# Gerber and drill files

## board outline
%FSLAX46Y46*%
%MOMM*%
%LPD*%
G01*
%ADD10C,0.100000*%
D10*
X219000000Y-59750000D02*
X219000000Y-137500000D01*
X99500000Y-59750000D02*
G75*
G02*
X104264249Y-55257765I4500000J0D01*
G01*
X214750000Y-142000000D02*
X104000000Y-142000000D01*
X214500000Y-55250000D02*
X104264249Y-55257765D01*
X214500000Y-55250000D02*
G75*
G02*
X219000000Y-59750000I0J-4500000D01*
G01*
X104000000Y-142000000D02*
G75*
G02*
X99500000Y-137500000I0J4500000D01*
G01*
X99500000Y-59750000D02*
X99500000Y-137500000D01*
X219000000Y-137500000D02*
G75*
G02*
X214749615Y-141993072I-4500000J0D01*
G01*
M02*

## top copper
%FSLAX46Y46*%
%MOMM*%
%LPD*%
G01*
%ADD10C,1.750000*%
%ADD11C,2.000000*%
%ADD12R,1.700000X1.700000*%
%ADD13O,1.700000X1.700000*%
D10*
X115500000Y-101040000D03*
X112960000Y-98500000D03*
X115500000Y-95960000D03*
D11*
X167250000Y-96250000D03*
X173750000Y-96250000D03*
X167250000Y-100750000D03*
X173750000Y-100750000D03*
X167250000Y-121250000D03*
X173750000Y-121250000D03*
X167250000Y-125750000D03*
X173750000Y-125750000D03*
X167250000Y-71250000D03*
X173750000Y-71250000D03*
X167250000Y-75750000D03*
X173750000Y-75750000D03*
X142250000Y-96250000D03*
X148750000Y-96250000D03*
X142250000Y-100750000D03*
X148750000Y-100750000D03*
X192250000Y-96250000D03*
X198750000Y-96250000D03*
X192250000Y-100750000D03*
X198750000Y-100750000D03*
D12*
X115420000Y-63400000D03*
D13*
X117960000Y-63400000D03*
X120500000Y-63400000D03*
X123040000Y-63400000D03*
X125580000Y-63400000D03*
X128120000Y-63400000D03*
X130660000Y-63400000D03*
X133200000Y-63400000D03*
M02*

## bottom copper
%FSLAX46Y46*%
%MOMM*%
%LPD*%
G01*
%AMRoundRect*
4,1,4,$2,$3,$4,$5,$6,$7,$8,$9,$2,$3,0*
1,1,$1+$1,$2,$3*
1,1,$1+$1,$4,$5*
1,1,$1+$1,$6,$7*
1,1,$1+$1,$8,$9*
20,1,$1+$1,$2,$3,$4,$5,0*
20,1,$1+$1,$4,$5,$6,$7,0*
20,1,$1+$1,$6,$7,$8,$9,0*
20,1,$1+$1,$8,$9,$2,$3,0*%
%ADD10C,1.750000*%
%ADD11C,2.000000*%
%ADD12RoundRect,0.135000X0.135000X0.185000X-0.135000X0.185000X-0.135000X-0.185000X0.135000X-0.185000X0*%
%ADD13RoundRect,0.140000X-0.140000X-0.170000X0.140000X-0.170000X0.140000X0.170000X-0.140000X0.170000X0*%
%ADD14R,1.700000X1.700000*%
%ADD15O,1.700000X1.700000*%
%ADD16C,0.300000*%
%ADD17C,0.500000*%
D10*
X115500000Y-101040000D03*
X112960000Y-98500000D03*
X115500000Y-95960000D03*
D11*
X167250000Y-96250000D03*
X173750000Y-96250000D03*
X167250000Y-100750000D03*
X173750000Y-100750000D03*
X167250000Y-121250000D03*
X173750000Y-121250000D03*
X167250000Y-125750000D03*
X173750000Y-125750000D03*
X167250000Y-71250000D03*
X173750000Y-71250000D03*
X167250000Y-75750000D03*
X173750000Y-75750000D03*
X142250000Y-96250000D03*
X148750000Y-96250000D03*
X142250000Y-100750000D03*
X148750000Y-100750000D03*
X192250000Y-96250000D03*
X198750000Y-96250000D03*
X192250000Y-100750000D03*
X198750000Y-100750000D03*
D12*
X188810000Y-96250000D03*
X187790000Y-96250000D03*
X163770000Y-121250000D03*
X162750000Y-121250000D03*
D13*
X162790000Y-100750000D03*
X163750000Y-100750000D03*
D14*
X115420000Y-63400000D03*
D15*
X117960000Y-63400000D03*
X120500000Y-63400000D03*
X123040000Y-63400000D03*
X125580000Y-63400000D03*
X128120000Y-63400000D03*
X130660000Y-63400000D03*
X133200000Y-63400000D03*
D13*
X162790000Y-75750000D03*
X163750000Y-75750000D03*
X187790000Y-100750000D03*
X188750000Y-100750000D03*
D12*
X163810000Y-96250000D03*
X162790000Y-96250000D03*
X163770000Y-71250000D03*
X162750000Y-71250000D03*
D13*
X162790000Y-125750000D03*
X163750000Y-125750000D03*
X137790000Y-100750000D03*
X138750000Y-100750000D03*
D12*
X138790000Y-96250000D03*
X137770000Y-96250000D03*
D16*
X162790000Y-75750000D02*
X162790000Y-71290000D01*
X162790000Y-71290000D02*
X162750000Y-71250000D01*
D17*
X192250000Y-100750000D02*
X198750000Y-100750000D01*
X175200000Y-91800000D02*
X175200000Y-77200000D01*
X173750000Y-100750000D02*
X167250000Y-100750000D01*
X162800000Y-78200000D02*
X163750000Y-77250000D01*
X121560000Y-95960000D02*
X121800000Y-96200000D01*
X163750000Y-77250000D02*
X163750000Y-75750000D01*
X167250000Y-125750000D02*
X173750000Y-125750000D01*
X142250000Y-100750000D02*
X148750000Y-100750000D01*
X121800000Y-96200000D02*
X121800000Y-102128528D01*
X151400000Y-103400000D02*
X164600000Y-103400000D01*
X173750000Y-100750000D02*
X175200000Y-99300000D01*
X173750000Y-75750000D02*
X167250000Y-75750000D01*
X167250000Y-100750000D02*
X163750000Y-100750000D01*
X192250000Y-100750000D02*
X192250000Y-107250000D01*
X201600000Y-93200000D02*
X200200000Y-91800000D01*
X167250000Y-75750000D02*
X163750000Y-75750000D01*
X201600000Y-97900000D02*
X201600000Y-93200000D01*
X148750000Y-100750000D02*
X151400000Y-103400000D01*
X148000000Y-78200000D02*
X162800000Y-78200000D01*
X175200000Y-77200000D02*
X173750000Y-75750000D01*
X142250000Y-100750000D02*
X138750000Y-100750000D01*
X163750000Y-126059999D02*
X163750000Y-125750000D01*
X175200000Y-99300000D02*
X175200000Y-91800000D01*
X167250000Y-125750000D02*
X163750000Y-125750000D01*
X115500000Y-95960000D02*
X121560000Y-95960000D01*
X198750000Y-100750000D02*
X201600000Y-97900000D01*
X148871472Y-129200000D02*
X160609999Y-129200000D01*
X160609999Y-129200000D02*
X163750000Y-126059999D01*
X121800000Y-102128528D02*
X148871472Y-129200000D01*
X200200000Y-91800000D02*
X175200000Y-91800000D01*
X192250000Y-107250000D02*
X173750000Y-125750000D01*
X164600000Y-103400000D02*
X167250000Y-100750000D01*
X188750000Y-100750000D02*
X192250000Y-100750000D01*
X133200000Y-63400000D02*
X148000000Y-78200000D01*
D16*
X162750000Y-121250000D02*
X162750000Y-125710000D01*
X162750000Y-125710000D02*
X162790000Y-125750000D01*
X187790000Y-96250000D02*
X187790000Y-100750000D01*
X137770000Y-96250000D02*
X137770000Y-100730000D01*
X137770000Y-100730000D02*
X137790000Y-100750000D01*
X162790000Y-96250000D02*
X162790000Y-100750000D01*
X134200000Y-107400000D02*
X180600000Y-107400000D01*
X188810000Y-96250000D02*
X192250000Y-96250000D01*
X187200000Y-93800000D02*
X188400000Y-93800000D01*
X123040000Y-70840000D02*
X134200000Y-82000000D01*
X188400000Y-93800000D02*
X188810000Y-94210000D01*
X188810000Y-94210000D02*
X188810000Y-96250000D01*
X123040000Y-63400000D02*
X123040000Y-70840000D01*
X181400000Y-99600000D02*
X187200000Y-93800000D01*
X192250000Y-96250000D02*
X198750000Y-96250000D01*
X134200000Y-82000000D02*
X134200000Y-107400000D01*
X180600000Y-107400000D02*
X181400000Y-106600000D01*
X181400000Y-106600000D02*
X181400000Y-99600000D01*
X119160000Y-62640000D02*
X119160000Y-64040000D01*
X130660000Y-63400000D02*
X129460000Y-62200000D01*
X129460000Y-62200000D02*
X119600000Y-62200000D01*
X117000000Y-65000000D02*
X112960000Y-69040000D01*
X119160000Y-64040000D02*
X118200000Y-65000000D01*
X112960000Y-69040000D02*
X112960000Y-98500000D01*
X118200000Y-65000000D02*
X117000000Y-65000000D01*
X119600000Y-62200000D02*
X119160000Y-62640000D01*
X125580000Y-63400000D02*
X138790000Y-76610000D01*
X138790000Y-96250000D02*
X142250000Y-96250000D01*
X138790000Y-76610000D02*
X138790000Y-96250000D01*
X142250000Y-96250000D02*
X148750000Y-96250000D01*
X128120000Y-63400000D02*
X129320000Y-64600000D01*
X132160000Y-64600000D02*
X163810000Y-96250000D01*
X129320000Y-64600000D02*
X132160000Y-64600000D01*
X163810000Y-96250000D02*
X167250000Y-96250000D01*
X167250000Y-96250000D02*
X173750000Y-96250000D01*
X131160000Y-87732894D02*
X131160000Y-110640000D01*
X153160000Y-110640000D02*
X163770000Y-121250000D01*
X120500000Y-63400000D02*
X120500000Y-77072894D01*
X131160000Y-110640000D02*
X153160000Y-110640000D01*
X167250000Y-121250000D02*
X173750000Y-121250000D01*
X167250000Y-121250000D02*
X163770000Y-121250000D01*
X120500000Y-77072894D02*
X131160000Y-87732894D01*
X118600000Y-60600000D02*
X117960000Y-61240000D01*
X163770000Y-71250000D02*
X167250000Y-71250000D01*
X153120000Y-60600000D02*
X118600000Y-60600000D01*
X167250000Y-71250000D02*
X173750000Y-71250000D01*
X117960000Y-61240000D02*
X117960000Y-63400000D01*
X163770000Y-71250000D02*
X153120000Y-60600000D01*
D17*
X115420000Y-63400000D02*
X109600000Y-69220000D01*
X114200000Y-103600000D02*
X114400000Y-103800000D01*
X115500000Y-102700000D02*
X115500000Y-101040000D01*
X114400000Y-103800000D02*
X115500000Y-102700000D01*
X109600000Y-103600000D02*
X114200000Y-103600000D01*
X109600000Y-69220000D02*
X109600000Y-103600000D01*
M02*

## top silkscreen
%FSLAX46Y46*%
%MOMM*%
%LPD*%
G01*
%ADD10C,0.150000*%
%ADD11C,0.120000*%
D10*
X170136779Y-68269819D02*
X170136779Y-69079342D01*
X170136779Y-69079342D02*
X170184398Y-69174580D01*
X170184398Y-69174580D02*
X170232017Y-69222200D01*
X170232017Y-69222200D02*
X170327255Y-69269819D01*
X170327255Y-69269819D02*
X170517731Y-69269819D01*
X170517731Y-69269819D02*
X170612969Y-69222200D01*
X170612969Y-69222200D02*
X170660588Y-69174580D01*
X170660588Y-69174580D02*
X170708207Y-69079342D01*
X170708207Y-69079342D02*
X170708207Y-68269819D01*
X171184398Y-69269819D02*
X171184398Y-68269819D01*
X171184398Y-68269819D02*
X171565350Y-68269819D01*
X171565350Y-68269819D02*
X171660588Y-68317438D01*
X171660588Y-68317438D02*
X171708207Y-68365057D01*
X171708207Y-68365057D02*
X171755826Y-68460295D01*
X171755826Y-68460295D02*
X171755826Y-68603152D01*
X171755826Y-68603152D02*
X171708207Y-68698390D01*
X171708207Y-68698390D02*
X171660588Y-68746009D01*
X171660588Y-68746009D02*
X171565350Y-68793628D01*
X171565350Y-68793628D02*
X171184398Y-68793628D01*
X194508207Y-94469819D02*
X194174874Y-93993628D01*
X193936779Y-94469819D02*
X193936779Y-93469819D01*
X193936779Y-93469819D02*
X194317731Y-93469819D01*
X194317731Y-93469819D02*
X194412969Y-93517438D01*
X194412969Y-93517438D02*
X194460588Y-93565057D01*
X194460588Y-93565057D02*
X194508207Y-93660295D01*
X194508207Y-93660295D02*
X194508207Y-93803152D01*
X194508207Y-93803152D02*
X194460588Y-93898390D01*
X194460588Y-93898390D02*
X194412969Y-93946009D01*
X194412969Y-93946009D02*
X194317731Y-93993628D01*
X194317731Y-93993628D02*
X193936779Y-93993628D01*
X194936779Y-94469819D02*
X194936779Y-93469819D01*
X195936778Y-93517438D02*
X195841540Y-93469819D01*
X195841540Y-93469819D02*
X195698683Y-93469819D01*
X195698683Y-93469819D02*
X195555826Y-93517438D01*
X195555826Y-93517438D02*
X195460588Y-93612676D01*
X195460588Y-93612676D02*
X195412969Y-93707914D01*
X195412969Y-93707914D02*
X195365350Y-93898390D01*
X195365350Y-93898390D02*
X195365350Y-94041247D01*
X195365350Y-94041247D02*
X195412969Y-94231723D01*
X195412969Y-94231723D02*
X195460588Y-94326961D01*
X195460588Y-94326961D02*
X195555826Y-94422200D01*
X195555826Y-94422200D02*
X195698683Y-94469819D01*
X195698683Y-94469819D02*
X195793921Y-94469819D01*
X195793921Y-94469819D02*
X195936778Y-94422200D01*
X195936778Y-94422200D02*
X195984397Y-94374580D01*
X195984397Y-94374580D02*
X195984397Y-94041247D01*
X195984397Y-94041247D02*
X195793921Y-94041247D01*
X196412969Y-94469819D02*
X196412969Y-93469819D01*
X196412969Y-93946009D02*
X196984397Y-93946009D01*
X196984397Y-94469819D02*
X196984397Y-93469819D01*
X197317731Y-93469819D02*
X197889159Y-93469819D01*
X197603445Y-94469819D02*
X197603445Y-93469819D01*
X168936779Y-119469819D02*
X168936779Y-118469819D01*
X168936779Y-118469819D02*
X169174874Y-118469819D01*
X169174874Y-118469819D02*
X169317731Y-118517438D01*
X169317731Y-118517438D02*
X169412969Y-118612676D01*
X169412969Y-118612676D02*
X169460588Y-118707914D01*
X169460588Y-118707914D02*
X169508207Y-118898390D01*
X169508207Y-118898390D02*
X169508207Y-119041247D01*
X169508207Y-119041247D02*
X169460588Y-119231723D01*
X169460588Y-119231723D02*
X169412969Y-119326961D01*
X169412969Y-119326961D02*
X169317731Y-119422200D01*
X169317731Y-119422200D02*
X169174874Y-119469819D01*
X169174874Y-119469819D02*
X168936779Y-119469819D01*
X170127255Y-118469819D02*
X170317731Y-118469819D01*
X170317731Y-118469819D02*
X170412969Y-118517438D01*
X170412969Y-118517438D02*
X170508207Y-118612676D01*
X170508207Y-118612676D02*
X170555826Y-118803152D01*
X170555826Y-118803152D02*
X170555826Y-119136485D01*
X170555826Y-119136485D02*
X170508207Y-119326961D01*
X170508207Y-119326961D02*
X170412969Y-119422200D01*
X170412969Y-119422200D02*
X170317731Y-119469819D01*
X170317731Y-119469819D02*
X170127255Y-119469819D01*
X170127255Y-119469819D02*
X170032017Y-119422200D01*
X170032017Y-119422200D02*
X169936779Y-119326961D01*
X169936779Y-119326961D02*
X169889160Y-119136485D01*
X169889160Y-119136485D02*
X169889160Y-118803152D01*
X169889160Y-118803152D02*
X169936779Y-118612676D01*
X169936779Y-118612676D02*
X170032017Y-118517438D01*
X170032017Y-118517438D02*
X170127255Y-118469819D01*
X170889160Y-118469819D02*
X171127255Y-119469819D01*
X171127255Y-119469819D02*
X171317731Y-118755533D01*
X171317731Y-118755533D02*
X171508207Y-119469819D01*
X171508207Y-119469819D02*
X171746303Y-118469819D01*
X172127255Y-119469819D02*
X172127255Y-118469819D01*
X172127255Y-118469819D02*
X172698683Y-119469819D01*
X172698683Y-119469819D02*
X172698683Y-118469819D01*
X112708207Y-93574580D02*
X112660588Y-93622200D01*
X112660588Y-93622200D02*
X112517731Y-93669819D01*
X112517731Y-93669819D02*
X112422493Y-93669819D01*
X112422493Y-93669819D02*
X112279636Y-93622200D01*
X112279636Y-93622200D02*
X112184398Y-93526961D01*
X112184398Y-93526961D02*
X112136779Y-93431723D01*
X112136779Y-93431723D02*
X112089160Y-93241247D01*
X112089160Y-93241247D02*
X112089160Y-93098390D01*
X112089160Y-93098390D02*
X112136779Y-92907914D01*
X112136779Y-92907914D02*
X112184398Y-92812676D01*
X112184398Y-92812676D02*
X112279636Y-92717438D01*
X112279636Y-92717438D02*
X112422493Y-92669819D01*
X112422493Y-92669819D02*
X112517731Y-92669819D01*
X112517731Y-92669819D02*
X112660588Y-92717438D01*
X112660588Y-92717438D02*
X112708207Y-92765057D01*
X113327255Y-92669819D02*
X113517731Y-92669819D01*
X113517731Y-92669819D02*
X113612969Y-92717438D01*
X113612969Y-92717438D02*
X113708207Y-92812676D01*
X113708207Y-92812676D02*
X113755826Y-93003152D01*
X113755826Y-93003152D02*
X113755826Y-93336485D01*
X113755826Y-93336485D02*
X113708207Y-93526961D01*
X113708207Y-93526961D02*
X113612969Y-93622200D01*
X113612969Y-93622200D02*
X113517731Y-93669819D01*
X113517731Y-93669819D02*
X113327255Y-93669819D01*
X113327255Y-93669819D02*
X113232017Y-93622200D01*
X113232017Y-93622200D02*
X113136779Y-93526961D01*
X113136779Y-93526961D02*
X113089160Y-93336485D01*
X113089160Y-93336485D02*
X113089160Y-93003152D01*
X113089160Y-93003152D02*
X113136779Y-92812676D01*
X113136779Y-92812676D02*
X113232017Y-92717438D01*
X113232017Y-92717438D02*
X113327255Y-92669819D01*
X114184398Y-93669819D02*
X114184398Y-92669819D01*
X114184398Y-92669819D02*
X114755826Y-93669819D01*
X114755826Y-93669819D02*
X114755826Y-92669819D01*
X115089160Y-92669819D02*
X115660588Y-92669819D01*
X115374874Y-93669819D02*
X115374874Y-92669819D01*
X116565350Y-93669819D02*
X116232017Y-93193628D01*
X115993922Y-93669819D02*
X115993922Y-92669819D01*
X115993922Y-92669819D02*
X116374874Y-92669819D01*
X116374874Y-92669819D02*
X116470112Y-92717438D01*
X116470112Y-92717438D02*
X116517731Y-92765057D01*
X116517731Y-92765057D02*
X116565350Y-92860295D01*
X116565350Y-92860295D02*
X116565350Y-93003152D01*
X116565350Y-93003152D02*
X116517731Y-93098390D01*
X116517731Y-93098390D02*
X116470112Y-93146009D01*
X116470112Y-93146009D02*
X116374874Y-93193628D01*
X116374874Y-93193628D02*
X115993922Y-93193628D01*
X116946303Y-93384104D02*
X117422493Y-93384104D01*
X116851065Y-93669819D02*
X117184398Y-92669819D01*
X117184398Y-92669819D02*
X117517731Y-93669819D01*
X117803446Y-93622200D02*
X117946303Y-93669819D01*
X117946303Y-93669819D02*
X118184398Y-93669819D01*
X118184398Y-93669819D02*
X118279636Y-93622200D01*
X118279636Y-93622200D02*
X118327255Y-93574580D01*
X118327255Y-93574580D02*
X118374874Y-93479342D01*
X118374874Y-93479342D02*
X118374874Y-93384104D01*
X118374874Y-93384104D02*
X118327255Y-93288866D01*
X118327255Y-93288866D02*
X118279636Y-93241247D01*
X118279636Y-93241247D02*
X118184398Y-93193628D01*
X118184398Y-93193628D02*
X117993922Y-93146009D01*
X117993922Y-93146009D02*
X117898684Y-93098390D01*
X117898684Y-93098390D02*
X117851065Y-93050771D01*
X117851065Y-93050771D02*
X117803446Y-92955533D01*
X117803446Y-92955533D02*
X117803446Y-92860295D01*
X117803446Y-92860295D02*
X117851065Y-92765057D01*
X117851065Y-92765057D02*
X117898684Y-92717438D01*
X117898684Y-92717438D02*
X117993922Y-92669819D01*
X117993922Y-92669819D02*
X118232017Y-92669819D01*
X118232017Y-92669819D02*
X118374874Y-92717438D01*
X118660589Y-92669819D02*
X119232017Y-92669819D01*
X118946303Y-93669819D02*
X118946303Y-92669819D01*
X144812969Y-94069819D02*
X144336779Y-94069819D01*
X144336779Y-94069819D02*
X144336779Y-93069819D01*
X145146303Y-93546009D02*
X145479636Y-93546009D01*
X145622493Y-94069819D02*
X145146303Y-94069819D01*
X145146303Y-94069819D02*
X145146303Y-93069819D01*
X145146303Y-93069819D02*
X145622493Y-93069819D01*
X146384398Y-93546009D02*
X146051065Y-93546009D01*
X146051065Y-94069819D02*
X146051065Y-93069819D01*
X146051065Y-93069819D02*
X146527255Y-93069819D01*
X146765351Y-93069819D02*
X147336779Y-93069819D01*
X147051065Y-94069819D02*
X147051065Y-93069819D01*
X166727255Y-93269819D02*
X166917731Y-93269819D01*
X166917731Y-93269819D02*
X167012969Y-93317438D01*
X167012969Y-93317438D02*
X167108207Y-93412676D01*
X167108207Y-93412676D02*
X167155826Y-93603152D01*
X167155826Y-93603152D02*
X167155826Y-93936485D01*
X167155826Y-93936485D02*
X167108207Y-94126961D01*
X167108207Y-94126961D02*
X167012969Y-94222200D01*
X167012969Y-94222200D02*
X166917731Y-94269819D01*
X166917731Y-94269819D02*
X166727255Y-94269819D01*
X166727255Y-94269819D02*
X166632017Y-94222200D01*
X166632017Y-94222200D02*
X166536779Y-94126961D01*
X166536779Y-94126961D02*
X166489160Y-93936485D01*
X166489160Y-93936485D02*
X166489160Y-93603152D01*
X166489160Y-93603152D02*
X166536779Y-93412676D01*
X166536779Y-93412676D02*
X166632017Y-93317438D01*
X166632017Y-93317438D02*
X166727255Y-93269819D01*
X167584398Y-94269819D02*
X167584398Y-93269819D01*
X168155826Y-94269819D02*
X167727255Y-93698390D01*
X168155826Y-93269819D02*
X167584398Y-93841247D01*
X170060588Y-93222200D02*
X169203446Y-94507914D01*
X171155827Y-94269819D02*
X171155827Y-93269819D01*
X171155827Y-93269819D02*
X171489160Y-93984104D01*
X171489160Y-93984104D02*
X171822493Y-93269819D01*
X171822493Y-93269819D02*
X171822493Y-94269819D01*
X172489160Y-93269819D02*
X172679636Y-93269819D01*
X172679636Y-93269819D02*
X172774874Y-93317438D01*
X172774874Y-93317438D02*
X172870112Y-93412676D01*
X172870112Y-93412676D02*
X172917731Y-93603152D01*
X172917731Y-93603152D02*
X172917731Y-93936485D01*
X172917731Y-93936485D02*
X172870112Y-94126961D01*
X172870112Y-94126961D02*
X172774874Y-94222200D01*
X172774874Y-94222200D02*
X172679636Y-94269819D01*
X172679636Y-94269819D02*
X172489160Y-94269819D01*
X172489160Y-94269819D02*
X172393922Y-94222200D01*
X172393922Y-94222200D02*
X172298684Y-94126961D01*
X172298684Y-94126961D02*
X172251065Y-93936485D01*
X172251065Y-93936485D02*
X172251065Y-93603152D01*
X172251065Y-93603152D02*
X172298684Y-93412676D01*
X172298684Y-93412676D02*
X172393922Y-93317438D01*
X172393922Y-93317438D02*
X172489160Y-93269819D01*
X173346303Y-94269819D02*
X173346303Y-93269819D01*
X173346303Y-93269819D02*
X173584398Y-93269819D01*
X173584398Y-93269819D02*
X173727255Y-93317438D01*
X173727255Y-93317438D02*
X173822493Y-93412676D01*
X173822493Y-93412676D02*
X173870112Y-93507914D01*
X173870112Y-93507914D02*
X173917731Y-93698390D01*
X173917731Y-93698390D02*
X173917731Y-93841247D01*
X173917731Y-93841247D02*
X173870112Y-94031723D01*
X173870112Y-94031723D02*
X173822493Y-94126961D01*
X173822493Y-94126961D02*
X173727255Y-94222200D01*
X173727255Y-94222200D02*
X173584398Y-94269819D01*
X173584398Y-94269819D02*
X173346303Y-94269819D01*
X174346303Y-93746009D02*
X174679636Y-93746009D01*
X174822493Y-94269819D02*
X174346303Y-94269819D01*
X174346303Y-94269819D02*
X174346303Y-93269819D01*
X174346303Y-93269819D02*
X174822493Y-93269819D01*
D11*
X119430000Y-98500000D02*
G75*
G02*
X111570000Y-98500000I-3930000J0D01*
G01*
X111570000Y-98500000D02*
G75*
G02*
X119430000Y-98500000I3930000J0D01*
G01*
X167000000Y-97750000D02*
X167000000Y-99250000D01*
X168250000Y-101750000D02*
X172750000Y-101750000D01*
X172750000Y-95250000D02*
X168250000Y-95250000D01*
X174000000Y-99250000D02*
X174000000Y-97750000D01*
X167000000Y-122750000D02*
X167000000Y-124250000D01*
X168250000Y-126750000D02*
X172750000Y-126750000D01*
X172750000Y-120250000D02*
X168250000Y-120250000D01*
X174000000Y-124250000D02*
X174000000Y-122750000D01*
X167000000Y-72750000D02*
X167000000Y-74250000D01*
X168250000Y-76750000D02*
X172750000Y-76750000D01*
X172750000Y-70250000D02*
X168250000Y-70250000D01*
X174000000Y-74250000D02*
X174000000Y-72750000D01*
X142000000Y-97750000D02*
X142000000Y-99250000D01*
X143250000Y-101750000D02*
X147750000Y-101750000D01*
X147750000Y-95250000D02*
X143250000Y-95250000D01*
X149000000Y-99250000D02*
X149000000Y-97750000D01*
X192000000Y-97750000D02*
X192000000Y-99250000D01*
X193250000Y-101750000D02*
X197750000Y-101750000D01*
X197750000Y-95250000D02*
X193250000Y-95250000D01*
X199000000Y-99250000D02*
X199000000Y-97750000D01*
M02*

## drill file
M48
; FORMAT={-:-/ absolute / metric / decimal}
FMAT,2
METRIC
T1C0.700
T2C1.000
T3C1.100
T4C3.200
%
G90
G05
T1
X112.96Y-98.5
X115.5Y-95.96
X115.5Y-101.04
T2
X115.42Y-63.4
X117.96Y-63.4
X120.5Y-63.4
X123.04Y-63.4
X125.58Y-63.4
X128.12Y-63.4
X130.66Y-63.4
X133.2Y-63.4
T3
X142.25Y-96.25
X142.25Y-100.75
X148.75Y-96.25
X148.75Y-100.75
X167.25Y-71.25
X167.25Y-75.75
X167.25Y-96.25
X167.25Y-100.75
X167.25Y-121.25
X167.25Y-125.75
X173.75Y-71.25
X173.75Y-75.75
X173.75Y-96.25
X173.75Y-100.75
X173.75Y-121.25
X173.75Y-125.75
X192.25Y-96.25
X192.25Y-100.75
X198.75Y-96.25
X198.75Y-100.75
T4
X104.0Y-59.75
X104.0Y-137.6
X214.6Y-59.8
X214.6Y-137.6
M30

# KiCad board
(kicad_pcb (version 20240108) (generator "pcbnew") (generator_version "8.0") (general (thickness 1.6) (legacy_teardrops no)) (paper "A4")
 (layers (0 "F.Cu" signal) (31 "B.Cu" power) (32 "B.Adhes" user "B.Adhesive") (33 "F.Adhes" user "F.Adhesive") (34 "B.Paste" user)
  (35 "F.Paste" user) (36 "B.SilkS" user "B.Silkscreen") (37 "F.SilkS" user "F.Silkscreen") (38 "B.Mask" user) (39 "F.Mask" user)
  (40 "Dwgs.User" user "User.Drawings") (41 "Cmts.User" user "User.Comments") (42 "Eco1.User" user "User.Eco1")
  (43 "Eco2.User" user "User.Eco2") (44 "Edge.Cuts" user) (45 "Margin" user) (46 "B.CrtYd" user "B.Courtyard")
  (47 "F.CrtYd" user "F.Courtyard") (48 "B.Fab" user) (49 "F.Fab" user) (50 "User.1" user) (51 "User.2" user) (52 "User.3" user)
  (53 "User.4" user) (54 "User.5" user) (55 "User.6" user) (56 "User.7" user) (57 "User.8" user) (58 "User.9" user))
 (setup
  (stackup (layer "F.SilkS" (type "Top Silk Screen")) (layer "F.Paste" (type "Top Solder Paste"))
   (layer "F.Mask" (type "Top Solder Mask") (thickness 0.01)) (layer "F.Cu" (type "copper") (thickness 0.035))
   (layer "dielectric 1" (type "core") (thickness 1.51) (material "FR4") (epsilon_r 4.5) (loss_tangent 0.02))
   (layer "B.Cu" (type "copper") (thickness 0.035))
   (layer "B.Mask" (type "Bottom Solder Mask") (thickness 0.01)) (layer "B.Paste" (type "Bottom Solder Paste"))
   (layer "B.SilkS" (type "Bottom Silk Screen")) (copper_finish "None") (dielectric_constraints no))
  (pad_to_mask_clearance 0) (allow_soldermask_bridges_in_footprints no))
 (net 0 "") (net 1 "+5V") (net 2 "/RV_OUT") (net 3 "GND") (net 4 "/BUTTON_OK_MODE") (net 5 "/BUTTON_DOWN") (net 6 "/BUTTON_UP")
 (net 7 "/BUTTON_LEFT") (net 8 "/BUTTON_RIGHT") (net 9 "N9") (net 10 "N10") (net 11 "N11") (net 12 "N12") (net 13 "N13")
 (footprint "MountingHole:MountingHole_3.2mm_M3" (layer "F.Cu") (at 104 137.6)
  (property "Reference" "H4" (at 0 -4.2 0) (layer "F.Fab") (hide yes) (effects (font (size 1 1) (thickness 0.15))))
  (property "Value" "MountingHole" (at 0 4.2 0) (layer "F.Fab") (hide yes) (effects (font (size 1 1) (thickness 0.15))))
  (pad "" np_thru_hole circle (at 0 0) (size 3.2 3.2) (drill 3.2) (layers "*.Cu" "*.Mask")))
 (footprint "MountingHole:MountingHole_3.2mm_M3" (layer "F.Cu") (at 104 59.75)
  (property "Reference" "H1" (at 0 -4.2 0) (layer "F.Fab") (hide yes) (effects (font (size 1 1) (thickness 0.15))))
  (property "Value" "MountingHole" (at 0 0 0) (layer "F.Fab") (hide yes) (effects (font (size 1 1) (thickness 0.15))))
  (pad "" np_thru_hole circle (at 0 0) (size 3.2 3.2) (drill 3.2) (layers "*.Cu" "*.Mask")))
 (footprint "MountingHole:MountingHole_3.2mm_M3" (layer "F.Cu") (at 214.6 137.6)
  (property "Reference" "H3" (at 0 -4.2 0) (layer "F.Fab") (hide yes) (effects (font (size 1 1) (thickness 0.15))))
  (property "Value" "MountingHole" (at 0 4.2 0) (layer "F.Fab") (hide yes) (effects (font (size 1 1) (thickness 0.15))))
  (pad "" np_thru_hole circle (at 0 0) (size 3.2 3.2) (drill 3.2) (layers "*.Cu" "*.Mask")))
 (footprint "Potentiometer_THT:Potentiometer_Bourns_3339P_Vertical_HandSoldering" (layer "F.Cu") (at 115.5 101.04)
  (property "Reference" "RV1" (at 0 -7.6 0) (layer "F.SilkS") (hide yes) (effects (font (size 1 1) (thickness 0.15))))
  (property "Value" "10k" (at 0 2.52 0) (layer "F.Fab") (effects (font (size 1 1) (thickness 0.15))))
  (fp_circle (center 0 -2.54) (end 3.93 -2.54) (stroke (width 0.12) (type solid)) (fill none) (layer "F.SilkS"))
  (pad "1" thru_hole circle (at 0 0) (size 1.75 1.75) (drill 0.7) (layers "*.Cu" "*.Mask") (remove_unused_layers no) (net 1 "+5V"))
  (pad "2" thru_hole circle (at -2.54 -2.54) (size 1.75 1.75) (drill 0.7) (layers "*.Cu" "*.Mask") (remove_unused_layers no)
   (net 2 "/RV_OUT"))
  (pad "3" thru_hole circle (at 0 -5.08) (size 1.75 1.75) (drill 0.7) (layers "*.Cu" "*.Mask") (remove_unused_layers no) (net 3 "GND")))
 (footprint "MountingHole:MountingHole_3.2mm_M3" (layer "F.Cu") (at 214.6 59.8)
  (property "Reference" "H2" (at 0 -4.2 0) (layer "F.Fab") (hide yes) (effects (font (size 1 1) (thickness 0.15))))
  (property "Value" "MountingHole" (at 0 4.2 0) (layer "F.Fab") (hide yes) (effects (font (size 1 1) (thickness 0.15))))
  (pad "" np_thru_hole circle (at 0 0) (size 3.2 3.2) (drill 3.2) (layers "*.Cu" "*.Mask")))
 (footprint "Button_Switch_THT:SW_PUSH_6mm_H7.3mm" (layer "F.Cu") (at 167.25 96.25)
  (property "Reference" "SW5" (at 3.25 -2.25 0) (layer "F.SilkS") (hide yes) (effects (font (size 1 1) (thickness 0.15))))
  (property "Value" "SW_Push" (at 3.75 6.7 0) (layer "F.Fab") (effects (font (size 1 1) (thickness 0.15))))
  (fp_line (start -0.25 1.5) (end -0.25 3) (stroke (width 0.12) (type solid)) (layer "F.SilkS"))
  (fp_line (start 1 5.5) (end 5.5 5.5) (stroke (width 0.12) (type solid)) (layer "F.SilkS"))
  (fp_line (start 5.5 -1) (end 1 -1) (stroke (width 0.12) (type solid)) (layer "F.SilkS"))
  (fp_line (start 6.75 3) (end 6.75 1.5) (stroke (width 0.12) (type solid)) (layer "F.SilkS"))
  (pad "1" thru_hole circle (at 0 0 90) (size 2 2) (drill 1.1) (layers "*.Cu" "*.Mask") (remove_unused_layers no) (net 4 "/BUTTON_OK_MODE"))
  (pad "1" thru_hole circle (at 6.5 0 90) (size 2 2) (drill 1.1) (layers "*.Cu" "*.Mask") (remove_unused_layers no)
   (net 4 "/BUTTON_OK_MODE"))
  (pad "2" thru_hole circle (at 0 4.5 90) (size 2 2) (drill 1.1) (layers "*.Cu" "*.Mask") (remove_unused_layers no) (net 3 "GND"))
  (pad "2" thru_hole circle (at 6.5 4.5 90) (size 2 2) (drill 1.1) (layers "*.Cu" "*.Mask") (remove_unused_layers no) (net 3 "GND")))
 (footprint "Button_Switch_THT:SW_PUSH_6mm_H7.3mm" (layer "F.Cu") (at 167.25 121.25)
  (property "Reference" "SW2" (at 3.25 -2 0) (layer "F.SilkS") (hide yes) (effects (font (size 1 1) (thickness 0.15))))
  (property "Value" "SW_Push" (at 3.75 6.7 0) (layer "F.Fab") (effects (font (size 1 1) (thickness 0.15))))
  (fp_line (start -0.25 1.5) (end -0.25 3) (stroke (width 0.12) (type solid)) (layer "F.SilkS"))
  (fp_line (start 1 5.5) (end 5.5 5.5) (stroke (width 0.12) (type solid)) (layer "F.SilkS"))
  (fp_line (start 5.5 -1) (end 1 -1) (stroke (width 0.12) (type solid)) (layer "F.SilkS"))
  (fp_line (start 6.75 3) (end 6.75 1.5) (stroke (width 0.12) (type solid)) (layer "F.SilkS"))
  (pad "1" thru_hole circle (at 0 0 90) (size 2 2) (drill 1.1) (layers "*.Cu" "*.Mask") (remove_unused_layers no) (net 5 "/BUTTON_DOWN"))
  (pad "1" thru_hole circle (at 6.5 0 90) (size 2 2) (drill 1.1) (layers "*.Cu" "*.Mask") (remove_unused_layers no) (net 5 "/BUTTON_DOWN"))
  (pad "2" thru_hole circle (at 0 4.5 90) (size 2 2) (drill 1.1) (layers "*.Cu" "*.Mask") (remove_unused_layers no) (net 3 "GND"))
  (pad "2" thru_hole circle (at 6.5 4.5 90) (size 2 2) (drill 1.1) (layers "*.Cu" "*.Mask") (remove_unused_layers no) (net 3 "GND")))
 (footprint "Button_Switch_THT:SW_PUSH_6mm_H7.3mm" (layer "F.Cu") (at 167.25 71.25)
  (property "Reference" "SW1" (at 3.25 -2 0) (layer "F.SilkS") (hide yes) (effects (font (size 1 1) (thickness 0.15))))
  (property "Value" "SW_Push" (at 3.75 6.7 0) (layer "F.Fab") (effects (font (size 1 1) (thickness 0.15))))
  (fp_line (start -0.25 1.5) (end -0.25 3) (stroke (width 0.12) (type solid)) (layer "F.SilkS"))
  (fp_line (start 1 5.5) (end 5.5 5.5) (stroke (width 0.12) (type solid)) (layer "F.SilkS"))
  (fp_line (start 5.5 -1) (end 1 -1) (stroke (width 0.12) (type solid)) (layer "F.SilkS"))
  (fp_line (start 6.75 3) (end 6.75 1.5) (stroke (width 0.12) (type solid)) (layer "F.SilkS"))
  (pad "1" thru_hole circle (at 0 0 90) (size 2 2) (drill 1.1) (layers "*.Cu" "*.Mask") (remove_unused_layers no) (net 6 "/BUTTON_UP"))
  (pad "1" thru_hole circle (at 6.5 0 90) (size 2 2) (drill 1.1) (layers "*.Cu" "*.Mask") (remove_unused_layers no) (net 6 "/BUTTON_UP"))
  (pad "2" thru_hole circle (at 0 4.5 90) (size 2 2) (drill 1.1) (layers "*.Cu" "*.Mask") (remove_unused_layers no) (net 3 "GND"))
  (pad "2" thru_hole circle (at 6.5 4.5 90) (size 2 2) (drill 1.1) (layers "*.Cu" "*.Mask") (remove_unused_layers no) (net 3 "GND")))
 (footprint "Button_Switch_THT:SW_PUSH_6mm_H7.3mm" (layer "F.Cu") (at 142.25 96.25)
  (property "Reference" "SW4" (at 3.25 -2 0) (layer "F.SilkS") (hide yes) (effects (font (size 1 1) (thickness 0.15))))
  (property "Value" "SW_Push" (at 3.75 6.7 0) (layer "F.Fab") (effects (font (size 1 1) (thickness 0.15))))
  (fp_line (start -0.25 1.5) (end -0.25 3) (stroke (width 0.12) (type solid)) (layer "F.SilkS"))
  (fp_line (start 1 5.5) (end 5.5 5.5) (stroke (width 0.12) (type solid)) (layer "F.SilkS"))
  (fp_line (start 5.5 -1) (end 1 -1) (stroke (width 0.12) (type solid)) (layer "F.SilkS"))
  (fp_line (start 6.75 3) (end 6.75 1.5) (stroke (width 0.12) (type solid)) (layer "F.SilkS"))
  (pad "1" thru_hole circle (at 0 0 90) (size 2 2) (drill 1.1) (layers "*.Cu" "*.Mask") (remove_unused_layers no) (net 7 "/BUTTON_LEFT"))
  (pad "1" thru_hole circle (at 6.5 0 90) (size 2 2) (drill 1.1) (layers "*.Cu" "*.Mask") (remove_unused_layers no) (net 7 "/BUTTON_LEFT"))
  (pad "2" thru_hole circle (at 0 4.5 90) (size 2 2) (drill 1.1) (layers "*.Cu" "*.Mask") (remove_unused_layers no) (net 3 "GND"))
  (pad "2" thru_hole circle (at 6.5 4.5 90) (size 2 2) (drill 1.1) (layers "*.Cu" "*.Mask") (remove_unused_layers no) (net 3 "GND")))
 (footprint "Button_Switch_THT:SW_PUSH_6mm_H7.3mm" (layer "F.Cu") (at 192.25 96.25)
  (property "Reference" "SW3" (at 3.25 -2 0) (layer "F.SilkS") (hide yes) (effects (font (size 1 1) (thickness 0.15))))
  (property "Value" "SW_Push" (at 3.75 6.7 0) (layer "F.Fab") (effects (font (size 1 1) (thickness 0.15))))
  (fp_line (start -0.25 1.5) (end -0.25 3) (stroke (width 0.12) (type solid)) (layer "F.SilkS"))
  (fp_line (start 1 5.5) (end 5.5 5.5) (stroke (width 0.12) (type solid)) (layer "F.SilkS"))
  (fp_line (start 5.5 -1) (end 1 -1) (stroke (width 0.12) (type solid)) (layer "F.SilkS"))
  (fp_line (start 6.75 3) (end 6.75 1.5) (stroke (width 0.12) (type solid)) (layer "F.SilkS"))
  (pad "1" thru_hole circle (at 0 0 90) (size 2 2) (drill 1.1) (layers "*.Cu" "*.Mask") (remove_unused_layers no) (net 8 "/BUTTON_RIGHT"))
  (pad "1" thru_hole circle (at 6.5 0 90) (size 2 2) (drill 1.1) (layers "*.Cu" "*.Mask") (remove_unused_layers no) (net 8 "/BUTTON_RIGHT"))
  (pad "2" thru_hole circle (at 0 4.5 90) (size 2 2) (drill 1.1) (layers "*.Cu" "*.Mask") (remove_unused_layers no) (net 3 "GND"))
  (pad "2" thru_hole circle (at 6.5 4.5 90) (size 2 2) (drill 1.1) (layers "*.Cu" "*.Mask") (remove_unused_layers no) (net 3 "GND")))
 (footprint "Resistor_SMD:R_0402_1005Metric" (layer "B.Cu") (at 188.3 96.25 180)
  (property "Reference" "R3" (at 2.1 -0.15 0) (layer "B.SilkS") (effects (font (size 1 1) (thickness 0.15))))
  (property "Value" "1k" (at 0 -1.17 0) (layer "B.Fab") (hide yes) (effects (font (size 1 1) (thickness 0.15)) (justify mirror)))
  (pad "1" smd roundrect (at -0.51 0 180) (size 0.54 0.64) (layers "B.Cu" "B.Paste" "B.Mask") (roundrect_rratio 0.25)
   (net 8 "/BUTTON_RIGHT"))
  (pad "2" smd roundrect (at 0.51 0 180) (size 0.54 0.64) (layers "B.Cu" "B.Paste" "B.Mask") (roundrect_rratio 0.25) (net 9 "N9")))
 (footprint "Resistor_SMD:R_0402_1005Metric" (layer "B.Cu") (at 163.26 121.25 180)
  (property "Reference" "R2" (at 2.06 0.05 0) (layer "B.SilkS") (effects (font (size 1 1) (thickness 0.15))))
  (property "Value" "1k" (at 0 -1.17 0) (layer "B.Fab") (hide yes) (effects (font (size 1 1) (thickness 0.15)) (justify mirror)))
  (pad "1" smd roundrect (at -0.51 0 180) (size 0.54 0.64) (layers "B.Cu" "B.Paste" "B.Mask") (roundrect_rratio 0.25) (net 5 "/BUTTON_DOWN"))
  (pad "2" smd roundrect (at 0.51 0 180) (size 0.54 0.64) (layers "B.Cu" "B.Paste" "B.Mask") (roundrect_rratio 0.25) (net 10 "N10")))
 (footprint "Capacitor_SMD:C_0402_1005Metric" (layer "B.Cu") (at 163.27 100.75)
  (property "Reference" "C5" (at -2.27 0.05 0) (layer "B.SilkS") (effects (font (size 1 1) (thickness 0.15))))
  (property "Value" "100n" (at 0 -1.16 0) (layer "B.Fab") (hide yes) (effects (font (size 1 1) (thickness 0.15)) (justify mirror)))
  (pad "1" smd roundrect (at -0.48 0) (size 0.56 0.62) (layers "B.Cu" "B.Paste" "B.Mask") (roundrect_rratio 0.25) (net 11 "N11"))
  (pad "2" smd roundrect (at 0.48 0) (size 0.56 0.62) (layers "B.Cu" "B.Paste" "B.Mask") (roundrect_rratio 0.25) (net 3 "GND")))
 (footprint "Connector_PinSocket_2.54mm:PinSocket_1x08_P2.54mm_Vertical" (layer "B.Cu") (at 115.42 63.4 -90)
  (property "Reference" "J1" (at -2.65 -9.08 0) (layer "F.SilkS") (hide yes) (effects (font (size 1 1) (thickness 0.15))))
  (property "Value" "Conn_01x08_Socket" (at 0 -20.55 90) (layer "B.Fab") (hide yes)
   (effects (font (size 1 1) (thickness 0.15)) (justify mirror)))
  (pad "1" thru_hole rect (at 0 0 270) (size 1.7 1.7) (drill 1) (layers "*.Cu" "*.Mask") (remove_unused_layers no) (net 1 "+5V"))
  (pad "2" thru_hole oval (at 0 -2.54 270) (size 1.7 1.7) (drill 1) (layers "*.Cu" "*.Mask") (remove_unused_layers no) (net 6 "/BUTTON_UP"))
  (pad "3" thru_hole oval (at 0 -5.08 270) (size 1.7 1.7) (drill 1) (layers "*.Cu" "*.Mask") (remove_unused_layers no)
   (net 5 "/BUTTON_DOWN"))
  (pad "4" thru_hole oval (at 0 -7.62 270) (size 1.7 1.7) (drill 1) (layers "*.Cu" "*.Mask") (remove_unused_layers no)
   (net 8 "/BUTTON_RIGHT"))
  (pad "5" thru_hole oval (at 0 -10.16 270) (size 1.7 1.7) (drill 1) (layers "*.Cu" "*.Mask") (remove_unused_layers no)
   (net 7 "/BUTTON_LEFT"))
  (pad "6" thru_hole oval (at 0 -12.7 270) (size 1.7 1.7) (drill 1) (layers "*.Cu" "*.Mask") (remove_unused_layers no)
   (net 4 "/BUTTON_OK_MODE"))
  (pad "7" thru_hole oval (at 0 -15.24 270) (size 1.7 1.7) (drill 1) (layers "*.Cu" "*.Mask") (remove_unused_layers no) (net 2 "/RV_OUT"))
  (pad "8" thru_hole oval (at 0 -17.78 270) (size 1.7 1.7) (drill 1) (layers "*.Cu" "*.Mask") (remove_unused_layers no) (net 3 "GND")))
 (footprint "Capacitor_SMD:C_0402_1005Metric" (layer "B.Cu") (at 163.27 75.75)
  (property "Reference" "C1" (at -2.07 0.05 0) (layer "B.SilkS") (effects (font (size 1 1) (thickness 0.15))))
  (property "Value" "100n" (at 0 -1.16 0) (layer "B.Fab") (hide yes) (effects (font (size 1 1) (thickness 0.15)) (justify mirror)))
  (pad "1" smd roundrect (at -0.48 0) (size 0.56 0.62) (layers "B.Cu" "B.Paste" "B.Mask") (roundrect_rratio 0.25) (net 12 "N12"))
  (pad "2" smd roundrect (at 0.48 0) (size 0.56 0.62) (layers "B.Cu" "B.Paste" "B.Mask") (roundrect_rratio 0.25) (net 3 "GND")))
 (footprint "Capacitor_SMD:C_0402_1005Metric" (layer "B.Cu") (at 188.27 100.75)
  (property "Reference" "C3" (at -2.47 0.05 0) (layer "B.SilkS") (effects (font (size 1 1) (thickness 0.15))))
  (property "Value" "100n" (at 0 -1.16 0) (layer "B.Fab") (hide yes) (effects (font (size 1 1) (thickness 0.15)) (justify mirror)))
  (pad "1" smd roundrect (at -0.48 0) (size 0.56 0.62) (layers "B.Cu" "B.Paste" "B.Mask") (roundrect_rratio 0.25) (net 9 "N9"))
  (pad "2" smd roundrect (at 0.48 0) (size 0.56 0.62) (layers "B.Cu" "B.Paste" "B.Mask") (roundrect_rratio 0.25) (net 3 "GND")))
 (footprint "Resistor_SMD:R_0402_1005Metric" (layer "B.Cu") (at 163.3 96.25 180)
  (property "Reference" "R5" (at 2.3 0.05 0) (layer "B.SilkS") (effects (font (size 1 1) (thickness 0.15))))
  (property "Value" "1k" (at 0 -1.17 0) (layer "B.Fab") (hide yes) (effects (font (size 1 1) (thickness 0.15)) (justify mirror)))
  (pad "1" smd roundrect (at -0.51 0 180) (size 0.54 0.64) (layers "B.Cu" "B.Paste" "B.Mask") (roundrect_rratio 0.25)
   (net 4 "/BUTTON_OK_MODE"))
  (pad "2" smd roundrect (at 0.51 0 180) (size 0.54 0.64) (layers "B.Cu" "B.Paste" "B.Mask") (roundrect_rratio 0.25) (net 11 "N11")))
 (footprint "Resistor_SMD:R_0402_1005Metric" (layer "B.Cu") (at 163.26 71.25 180)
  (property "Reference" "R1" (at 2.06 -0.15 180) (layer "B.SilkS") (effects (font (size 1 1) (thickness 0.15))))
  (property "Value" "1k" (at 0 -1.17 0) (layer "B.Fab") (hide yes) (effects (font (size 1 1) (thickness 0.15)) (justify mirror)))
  (pad "1" smd roundrect (at -0.51 0 180) (size 0.54 0.64) (layers "B.Cu" "B.Paste" "B.Mask") (roundrect_rratio 0.25) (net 6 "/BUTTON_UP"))
  (pad "2" smd roundrect (at 0.51 0 180) (size 0.54 0.64) (layers "B.Cu" "B.Paste" "B.Mask") (roundrect_rratio 0.25) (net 12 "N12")))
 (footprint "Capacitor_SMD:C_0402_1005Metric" (layer "B.Cu") (at 163.27 125.75)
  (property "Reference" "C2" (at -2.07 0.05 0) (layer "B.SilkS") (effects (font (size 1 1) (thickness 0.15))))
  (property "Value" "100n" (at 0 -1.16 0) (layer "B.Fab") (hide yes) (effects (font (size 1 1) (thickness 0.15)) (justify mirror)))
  (pad "1" smd roundrect (at -0.48 0) (size 0.56 0.62) (layers "B.Cu" "B.Paste" "B.Mask") (roundrect_rratio 0.25) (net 10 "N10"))
  (pad "2" smd roundrect (at 0.48 0) (size 0.56 0.62) (layers "B.Cu" "B.Paste" "B.Mask") (roundrect_rratio 0.25) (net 3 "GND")))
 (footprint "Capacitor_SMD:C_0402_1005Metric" (layer "B.Cu") (at 138.27 100.75)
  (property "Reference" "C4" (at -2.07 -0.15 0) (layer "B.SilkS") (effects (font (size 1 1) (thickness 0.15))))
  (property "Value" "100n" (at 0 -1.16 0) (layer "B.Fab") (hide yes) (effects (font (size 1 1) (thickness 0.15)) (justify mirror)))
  (pad "1" smd roundrect (at -0.48 0) (size 0.56 0.62) (layers "B.Cu" "B.Paste" "B.Mask") (roundrect_rratio 0.25) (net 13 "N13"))
  (pad "2" smd roundrect (at 0.48 0) (size 0.56 0.62) (layers "B.Cu" "B.Paste" "B.Mask") (roundrect_rratio 0.25) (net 3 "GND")))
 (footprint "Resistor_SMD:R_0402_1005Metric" (layer "B.Cu") (at 138.28 96.25 180)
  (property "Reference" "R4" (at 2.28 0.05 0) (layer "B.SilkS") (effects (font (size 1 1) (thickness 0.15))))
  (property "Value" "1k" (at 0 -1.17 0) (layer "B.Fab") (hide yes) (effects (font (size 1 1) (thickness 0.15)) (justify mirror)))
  (pad "1" smd roundrect (at -0.51 0 180) (size 0.54 0.64) (layers "B.Cu" "B.Paste" "B.Mask") (roundrect_rratio 0.25) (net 7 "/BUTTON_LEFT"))
  (pad "2" smd roundrect (at 0.51 0 180) (size 0.54 0.64) (layers "B.Cu" "B.Paste" "B.Mask") (roundrect_rratio 0.25) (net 13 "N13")))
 (gr_line (start 219 59.75) (end 219 137.5) (stroke (width 0.1) (type default)) (layer "Edge.Cuts"))
 (gr_arc (start 99.5 59.75) (mid 100.912859 56.475926) (end 104.264249 55.257765) (stroke (width 0.1) (type default)) (layer "Edge.Cuts"))
 (gr_line (start 214.75 142) (end 104 142) (stroke (width 0.1) (type default)) (layer "Edge.Cuts"))
 (gr_line (start 214.5 55.25) (end 104.264249 55.257765) (stroke (width 0.1) (type default)) (layer "Edge.Cuts"))
 (gr_arc (start 214.5 55.25) (mid 217.681981 56.568019) (end 219 59.75) (stroke (width 0.1) (type default)) (layer "Edge.Cuts"))
 (gr_arc (start 104 142) (mid 100.818019 140.681981) (end 99.5 137.5) (stroke (width 0.1) (type default)) (layer "Edge.Cuts"))
 (gr_line (start 99.5 59.75) (end 99.5 137.5) (stroke (width 0.1) (type default)) (layer "Edge.Cuts"))
 (gr_arc (start 219 137.5) (mid 217.769042 140.592469) (end 214.749615 141.993072) (stroke (width 0.1) (type default)) (layer "Edge.Cuts"))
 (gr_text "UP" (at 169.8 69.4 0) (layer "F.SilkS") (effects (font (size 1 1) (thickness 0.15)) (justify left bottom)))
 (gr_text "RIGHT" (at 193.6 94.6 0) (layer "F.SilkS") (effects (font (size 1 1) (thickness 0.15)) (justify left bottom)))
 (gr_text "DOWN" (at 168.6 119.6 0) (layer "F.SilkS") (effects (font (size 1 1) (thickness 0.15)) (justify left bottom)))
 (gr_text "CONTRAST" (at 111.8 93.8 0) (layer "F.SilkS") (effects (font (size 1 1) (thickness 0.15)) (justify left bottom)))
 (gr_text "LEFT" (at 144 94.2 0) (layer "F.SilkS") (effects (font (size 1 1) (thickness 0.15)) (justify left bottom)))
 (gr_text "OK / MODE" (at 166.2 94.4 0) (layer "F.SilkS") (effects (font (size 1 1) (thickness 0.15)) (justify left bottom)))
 (segment (start 162.79 75.75) (end 162.79 71.29) (width 0.3) (layer "B.Cu") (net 12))
 (segment (start 162.79 71.29) (end 162.75 71.25) (width 0.3) (layer "B.Cu") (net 12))
 (segment (start 192.25 100.75) (end 198.75 100.75) (width 0.5) (layer "B.Cu") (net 3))
 (segment (start 175.2 91.8) (end 175.2 77.2) (width 0.5) (layer "B.Cu") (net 3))
 (segment (start 173.75 100.75) (end 167.25 100.75) (width 0.5) (layer "B.Cu") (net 3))
 (segment (start 162.8 78.2) (end 163.75 77.25) (width 0.5) (layer "B.Cu") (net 3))
 (segment (start 121.56 95.96) (end 121.8 96.2) (width 0.5) (layer "B.Cu") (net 3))
 (segment (start 163.75 77.25) (end 163.75 75.75) (width 0.5) (layer "B.Cu") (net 3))
 (segment (start 167.25 125.75) (end 173.75 125.75) (width 0.5) (layer "B.Cu") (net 3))
 (segment (start 142.25 100.75) (end 148.75 100.75) (width 0.5) (layer "B.Cu") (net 3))
 (segment (start 121.8 96.2) (end 121.8 102.128528) (width 0.5) (layer "B.Cu") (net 3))
 (segment (start 151.4 103.4) (end 164.6 103.4) (width 0.5) (layer "B.Cu") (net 3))
 (segment (start 173.75 100.75) (end 175.2 99.3) (width 0.5) (layer "B.Cu") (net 3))
 (segment (start 173.75 75.75) (end 167.25 75.75) (width 0.5) (layer "B.Cu") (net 3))
 (segment (start 167.25 100.75) (end 163.75 100.75) (width 0.5) (layer "B.Cu") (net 3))
 (segment (start 192.25 100.75) (end 192.25 107.25) (width 0.5) (layer "B.Cu") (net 3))
 (segment (start 201.6 93.2) (end 200.2 91.8) (width 0.5) (layer "B.Cu") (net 3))
 (segment (start 167.25 75.75) (end 163.75 75.75) (width 0.5) (layer "B.Cu") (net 3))
 (segment (start 201.6 97.9) (end 201.6 93.2) (width 0.5) (layer "B.Cu") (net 3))
 (segment (start 148.75 100.75) (end 151.4 103.4) (width 0.5) (layer "B.Cu") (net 3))
 (segment (start 148 78.2) (end 162.8 78.2) (width 0.5) (layer "B.Cu") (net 3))
 (segment (start 175.2 77.2) (end 173.75 75.75) (width 0.5) (layer "B.Cu") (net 3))
 (segment (start 142.25 100.75) (end 138.75 100.75) (width 0.5) (layer "B.Cu") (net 3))
 (segment (start 163.75 126.059999) (end 163.75 125.75) (width 0.5) (layer "B.Cu") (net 3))
 (segment (start 175.2 99.3) (end 175.2 91.8) (width 0.5) (layer "B.Cu") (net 3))
 (segment (start 167.25 125.75) (end 163.75 125.75) (width 0.5) (layer "B.Cu") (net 3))
 (segment (start 115.5 95.96) (end 121.56 95.96) (width 0.5) (layer "B.Cu") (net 3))
 (segment (start 198.75 100.75) (end 201.6 97.9) (width 0.5) (layer "B.Cu") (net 3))
 (segment (start 148.871472 129.2) (end 160.609999 129.2) (width 0.5) (layer "B.Cu") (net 3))
 (segment (start 160.609999 129.2) (end 163.75 126.059999) (width 0.5) (layer "B.Cu") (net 3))
 (segment (start 121.8 102.128528) (end 148.871472 129.2) (width 0.5) (layer "B.Cu") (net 3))
 (segment (start 200.2 91.8) (end 175.2 91.8) (width 0.5) (layer "B.Cu") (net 3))
 (segment (start 192.25 107.25) (end 173.75 125.75) (width 0.5) (layer "B.Cu") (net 3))
 (segment (start 164.6 103.4) (end 167.25 100.75) (width 0.5) (layer "B.Cu") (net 3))
 (segment (start 188.75 100.75) (end 192.25 100.75) (width 0.5) (layer "B.Cu") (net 3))
 (segment (start 133.2 63.4) (end 148 78.2) (width 0.5) (layer "B.Cu") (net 3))
 (segment (start 162.75 121.25) (end 162.75 125.71) (width 0.3) (layer "B.Cu") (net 10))
 (segment (start 162.75 125.71) (end 162.79 125.75) (width 0.3) (layer "B.Cu") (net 10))
 (segment (start 187.79 96.25) (end 187.79 100.75) (width 0.3) (layer "B.Cu") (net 9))
 (segment (start 137.77 96.25) (end 137.77 100.73) (width 0.3) (layer "B.Cu") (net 13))
 (segment (start 137.77 100.73) (end 137.79 100.75) (width 0.3) (layer "B.Cu") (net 13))
 (segment (start 162.79 96.25) (end 162.79 100.75) (width 0.3) (layer "B.Cu") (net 11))
 (segment (start 134.2 107.4) (end 180.6 107.4) (width 0.3) (layer "B.Cu") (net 8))
 (segment (start 188.81 96.25) (end 192.25 96.25) (width 0.3) (layer "B.Cu") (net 8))
 (segment (start 187.2 93.8) (end 188.4 93.8) (width 0.3) (layer "B.Cu") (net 8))
 (segment (start 123.04 70.84) (end 134.2 82) (width 0.3) (layer "B.Cu") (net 8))
 (segment (start 188.4 93.8) (end 188.81 94.21) (width 0.3) (layer "B.Cu") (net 8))
 (segment (start 188.81 94.21) (end 188.81 96.25) (width 0.3) (layer "B.Cu") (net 8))
 (segment (start 123.04 63.4) (end 123.04 70.84) (width 0.3) (layer "B.Cu") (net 8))
 (segment (start 181.4 99.6) (end 187.2 93.8) (width 0.3) (layer "B.Cu") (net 8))
 (segment (start 192.25 96.25) (end 198.75 96.25) (width 0.3) (layer "B.Cu") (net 8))
 (segment (start 134.2 82) (end 134.2 107.4) (width 0.3) (layer "B.Cu") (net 8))
 (segment (start 180.6 107.4) (end 181.4 106.6) (width 0.3) (layer "B.Cu") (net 8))
 (segment (start 181.4 106.6) (end 181.4 99.6) (width 0.3) (layer "B.Cu") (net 8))
 (segment (start 119.16 62.64) (end 119.16 64.04) (width 0.3) (layer "B.Cu") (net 2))
 (segment (start 130.66 63.4) (end 129.46 62.2) (width 0.3) (layer "B.Cu") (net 2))
 (segment (start 129.46 62.2) (end 119.6 62.2) (width 0.3) (layer "B.Cu") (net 2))
 (segment (start 117 65) (end 112.96 69.04) (width 0.3) (layer "B.Cu") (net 2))
 (segment (start 119.16 64.04) (end 118.2 65) (width 0.3) (layer "B.Cu") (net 2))
 (segment (start 112.96 69.04) (end 112.96 98.5) (width 0.3) (layer "B.Cu") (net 2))
 (segment (start 118.2 65) (end 117 65) (width 0.3) (layer "B.Cu") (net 2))
 (segment (start 119.6 62.2) (end 119.16 62.64) (width 0.3) (layer "B.Cu") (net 2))
 (segment (start 125.58 63.4) (end 138.79 76.61) (width 0.3) (layer "B.Cu") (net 7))
 (segment (start 138.79 96.25) (end 142.25 96.25) (width 0.3) (layer "B.Cu") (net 7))
 (segment (start 138.79 76.61) (end 138.79 96.25) (width 0.3) (layer "B.Cu") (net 7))
 (segment (start 142.25 96.25) (end 148.75 96.25) (width 0.3) (layer "B.Cu") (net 7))
 (segment (start 128.12 63.4) (end 129.32 64.6) (width 0.3) (layer "B.Cu") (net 4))
 (segment (start 132.16 64.6) (end 163.81 96.25) (width 0.3) (layer "B.Cu") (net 4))
 (segment (start 129.32 64.6) (end 132.16 64.6) (width 0.3) (layer "B.Cu") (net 4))
 (segment (start 163.81 96.25) (end 167.25 96.25) (width 0.3) (layer "B.Cu") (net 4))
 (segment (start 167.25 96.25) (end 173.75 96.25) (width 0.3) (layer "B.Cu") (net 4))
 (segment (start 131.16 87.732894) (end 131.16 110.64) (width 0.3) (layer "B.Cu") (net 5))
 (segment (start 153.16 110.64) (end 163.77 121.25) (width 0.3) (layer "B.Cu") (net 5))
 (segment (start 120.5 63.4) (end 120.5 77.072894) (width 0.3) (layer "B.Cu") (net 5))
 (segment (start 131.16 110.64) (end 153.16 110.64) (width 0.3) (layer "B.Cu") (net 5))
 (segment (start 167.25 121.25) (end 173.75 121.25) (width 0.3) (layer "B.Cu") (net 5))
 (segment (start 167.25 121.25) (end 163.77 121.25) (width 0.3) (layer "B.Cu") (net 5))
 (segment (start 120.5 77.072894) (end 131.16 87.732894) (width 0.3) (layer "B.Cu") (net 5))
 (segment (start 118.6 60.6) (end 117.96 61.24) (width 0.3) (layer "B.Cu") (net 6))
 (segment (start 163.77 71.25) (end 167.25 71.25) (width 0.3) (layer "B.Cu") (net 6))
 (segment (start 153.12 60.6) (end 118.6 60.6) (width 0.3) (layer "B.Cu") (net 6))
 (segment (start 167.25 71.25) (end 173.75 71.25) (width 0.3) (layer "B.Cu") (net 6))
 (segment (start 117.96 61.24) (end 117.96 63.4) (width 0.3) (layer "B.Cu") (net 6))
 (segment (start 163.77 71.25) (end 153.12 60.6) (width 0.3) (layer "B.Cu") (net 6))
 (segment (start 115.42 63.4) (end 109.6 69.22) (width 0.5) (layer "B.Cu") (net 1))
 (segment (start 114.2 103.6) (end 114.4 103.8) (width 0.5) (layer "B.Cu") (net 1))
 (segment (start 115.5 102.7) (end 115.5 101.04) (width 0.5) (layer "B.Cu") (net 1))
 (segment (start 114.4 103.8) (end 115.5 102.7) (width 0.5) (layer "B.Cu") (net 1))
 (segment (start 109.6 103.6) (end 114.2 103.6) (width 0.5) (layer "B.Cu") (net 1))
 (segment (start 109.6 69.22) (end 109.6 103.6) (width 0.5) (layer "B.Cu") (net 1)))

